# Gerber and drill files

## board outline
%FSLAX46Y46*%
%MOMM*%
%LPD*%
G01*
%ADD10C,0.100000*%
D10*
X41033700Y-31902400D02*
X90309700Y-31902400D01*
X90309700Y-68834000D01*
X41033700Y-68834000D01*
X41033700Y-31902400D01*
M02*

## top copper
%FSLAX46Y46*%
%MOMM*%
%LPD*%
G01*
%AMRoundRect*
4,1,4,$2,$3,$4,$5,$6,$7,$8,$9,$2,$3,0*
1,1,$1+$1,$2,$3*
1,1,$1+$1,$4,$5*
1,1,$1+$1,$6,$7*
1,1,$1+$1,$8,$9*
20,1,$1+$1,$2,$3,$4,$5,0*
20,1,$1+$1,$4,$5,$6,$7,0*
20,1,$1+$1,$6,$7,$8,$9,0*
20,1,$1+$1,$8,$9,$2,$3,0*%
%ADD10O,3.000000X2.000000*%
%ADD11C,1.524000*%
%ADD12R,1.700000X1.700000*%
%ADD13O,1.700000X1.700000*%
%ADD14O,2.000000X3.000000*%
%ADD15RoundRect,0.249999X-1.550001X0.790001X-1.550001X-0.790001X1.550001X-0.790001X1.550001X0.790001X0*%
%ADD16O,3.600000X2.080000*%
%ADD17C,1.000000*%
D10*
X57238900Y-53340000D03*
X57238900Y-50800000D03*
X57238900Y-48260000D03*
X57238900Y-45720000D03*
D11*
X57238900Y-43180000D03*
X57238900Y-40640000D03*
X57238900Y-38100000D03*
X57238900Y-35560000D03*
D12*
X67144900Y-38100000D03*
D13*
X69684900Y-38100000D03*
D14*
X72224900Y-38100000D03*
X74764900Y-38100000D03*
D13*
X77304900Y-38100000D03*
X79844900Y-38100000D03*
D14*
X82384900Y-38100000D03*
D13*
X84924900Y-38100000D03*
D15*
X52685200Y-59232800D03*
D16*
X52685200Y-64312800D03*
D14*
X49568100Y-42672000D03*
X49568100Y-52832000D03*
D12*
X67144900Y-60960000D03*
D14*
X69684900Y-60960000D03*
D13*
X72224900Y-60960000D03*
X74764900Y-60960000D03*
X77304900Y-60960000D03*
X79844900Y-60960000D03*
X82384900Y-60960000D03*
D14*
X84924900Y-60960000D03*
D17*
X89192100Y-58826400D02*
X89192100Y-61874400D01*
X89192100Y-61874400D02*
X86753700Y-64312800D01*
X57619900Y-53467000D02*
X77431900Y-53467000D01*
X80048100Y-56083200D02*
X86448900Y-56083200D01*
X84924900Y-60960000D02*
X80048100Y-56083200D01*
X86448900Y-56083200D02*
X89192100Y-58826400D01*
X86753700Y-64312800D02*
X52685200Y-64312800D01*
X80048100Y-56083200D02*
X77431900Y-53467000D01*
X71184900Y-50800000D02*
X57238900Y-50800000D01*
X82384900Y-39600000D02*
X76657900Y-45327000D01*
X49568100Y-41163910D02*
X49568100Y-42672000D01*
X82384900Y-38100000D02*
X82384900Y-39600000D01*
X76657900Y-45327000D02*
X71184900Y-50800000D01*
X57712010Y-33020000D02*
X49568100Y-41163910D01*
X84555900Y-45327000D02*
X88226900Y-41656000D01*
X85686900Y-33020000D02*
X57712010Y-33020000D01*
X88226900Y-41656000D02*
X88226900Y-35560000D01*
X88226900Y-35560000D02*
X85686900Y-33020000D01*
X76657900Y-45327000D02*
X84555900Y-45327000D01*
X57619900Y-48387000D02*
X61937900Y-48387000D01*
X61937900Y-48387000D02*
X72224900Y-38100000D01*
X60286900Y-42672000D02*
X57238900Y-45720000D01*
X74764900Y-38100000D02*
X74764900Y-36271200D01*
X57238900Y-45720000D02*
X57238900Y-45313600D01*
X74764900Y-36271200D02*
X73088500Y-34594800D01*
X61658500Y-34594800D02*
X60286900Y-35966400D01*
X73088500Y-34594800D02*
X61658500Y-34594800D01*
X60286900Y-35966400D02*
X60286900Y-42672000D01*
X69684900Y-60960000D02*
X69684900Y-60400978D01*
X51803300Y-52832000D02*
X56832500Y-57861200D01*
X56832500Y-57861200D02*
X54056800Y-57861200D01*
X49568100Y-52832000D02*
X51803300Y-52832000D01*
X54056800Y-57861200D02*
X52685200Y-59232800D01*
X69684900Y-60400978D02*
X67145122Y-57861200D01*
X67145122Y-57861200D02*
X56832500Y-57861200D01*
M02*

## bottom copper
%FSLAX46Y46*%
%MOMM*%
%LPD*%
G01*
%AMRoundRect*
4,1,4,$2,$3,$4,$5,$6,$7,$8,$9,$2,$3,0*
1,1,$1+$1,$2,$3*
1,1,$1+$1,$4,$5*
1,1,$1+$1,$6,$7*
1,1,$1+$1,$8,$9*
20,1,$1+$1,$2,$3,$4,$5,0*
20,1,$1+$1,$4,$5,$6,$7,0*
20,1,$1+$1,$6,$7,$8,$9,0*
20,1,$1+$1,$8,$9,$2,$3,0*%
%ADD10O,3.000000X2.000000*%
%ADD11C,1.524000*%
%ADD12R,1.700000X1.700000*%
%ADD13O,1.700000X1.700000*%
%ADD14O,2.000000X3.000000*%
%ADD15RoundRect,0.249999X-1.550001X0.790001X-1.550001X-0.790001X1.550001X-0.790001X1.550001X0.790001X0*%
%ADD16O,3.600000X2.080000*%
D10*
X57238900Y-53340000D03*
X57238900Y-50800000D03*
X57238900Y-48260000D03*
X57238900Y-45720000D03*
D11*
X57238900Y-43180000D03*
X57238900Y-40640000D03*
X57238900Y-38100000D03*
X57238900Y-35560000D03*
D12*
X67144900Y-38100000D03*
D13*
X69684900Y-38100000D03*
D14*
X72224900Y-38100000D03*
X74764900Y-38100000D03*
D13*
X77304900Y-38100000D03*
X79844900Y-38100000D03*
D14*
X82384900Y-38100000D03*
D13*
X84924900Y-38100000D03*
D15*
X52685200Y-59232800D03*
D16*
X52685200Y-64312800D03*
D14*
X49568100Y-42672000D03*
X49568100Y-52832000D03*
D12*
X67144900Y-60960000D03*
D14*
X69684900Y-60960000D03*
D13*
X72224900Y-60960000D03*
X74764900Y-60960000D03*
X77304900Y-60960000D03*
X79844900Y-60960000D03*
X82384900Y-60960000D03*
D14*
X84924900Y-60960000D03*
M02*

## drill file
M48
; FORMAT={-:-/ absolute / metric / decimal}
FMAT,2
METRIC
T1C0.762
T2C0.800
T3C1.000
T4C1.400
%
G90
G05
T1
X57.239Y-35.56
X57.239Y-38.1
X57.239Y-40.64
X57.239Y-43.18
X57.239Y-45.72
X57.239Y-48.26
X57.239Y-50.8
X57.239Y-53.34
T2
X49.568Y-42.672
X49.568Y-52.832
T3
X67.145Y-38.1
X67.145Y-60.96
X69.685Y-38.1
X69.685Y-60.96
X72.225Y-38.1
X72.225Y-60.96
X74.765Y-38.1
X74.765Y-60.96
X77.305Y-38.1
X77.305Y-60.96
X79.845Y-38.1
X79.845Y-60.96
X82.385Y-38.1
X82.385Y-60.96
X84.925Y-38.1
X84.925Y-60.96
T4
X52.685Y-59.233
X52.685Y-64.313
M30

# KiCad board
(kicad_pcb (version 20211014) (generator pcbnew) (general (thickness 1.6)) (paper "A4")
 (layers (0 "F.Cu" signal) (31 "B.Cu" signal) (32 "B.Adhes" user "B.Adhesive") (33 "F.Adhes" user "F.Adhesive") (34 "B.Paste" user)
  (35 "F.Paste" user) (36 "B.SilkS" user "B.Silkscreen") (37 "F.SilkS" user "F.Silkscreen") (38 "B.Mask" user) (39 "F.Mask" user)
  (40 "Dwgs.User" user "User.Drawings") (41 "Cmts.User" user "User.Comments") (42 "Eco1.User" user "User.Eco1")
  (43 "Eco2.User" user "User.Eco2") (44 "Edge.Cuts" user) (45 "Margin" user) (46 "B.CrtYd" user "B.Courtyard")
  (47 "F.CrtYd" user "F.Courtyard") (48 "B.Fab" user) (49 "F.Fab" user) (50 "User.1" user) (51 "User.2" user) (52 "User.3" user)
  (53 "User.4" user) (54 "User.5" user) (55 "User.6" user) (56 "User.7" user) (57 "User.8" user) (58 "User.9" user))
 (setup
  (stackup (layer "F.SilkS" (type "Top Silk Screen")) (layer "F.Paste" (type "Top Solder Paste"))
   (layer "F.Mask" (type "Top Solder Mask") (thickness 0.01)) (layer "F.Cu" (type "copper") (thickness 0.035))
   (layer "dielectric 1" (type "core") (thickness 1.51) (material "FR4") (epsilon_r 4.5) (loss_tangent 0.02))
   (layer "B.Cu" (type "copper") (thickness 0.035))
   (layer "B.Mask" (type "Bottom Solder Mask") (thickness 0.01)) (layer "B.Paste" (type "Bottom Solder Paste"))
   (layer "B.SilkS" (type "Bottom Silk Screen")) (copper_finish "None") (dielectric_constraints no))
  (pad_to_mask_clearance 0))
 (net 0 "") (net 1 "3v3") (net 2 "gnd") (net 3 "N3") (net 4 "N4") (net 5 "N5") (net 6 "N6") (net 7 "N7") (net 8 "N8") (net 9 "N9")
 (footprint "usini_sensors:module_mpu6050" (layer "F.Cu") (at 57.2389 35.56 180)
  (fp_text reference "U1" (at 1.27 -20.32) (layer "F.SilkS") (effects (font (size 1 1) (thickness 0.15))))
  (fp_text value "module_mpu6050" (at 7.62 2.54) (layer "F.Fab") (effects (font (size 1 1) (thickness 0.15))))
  (pad "1" thru_hole oval locked (at 0 -17.78 180) (size 3 2) (drill 0.762) (layers *.Cu *.Mask) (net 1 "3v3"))
  (pad "2" thru_hole oval locked (at 0 -15.24 180) (size 3 2) (drill 0.762) (layers *.Cu *.Mask) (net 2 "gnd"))
  (pad "3" thru_hole oval locked (at 0 -12.7 180) (size 3 2) (drill 0.762) (layers *.Cu *.Mask) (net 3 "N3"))
  (pad "4" thru_hole oval locked (at 0 -10.16 180) (size 3 2) (drill 0.762) (layers *.Cu *.Mask) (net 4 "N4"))
  (pad "5" thru_hole circle locked (at 0 -7.62 180) (size 1.524 1.524) (drill 0.762) (layers *.Cu *.Mask) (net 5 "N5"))
  (pad "6" thru_hole circle locked (at 0 -5.08 180) (size 1.524 1.524) (drill 0.762) (layers *.Cu *.Mask) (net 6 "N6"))
  (pad "7" thru_hole circle locked (at 0 -2.54 180) (size 1.524 1.524) (drill 0.762) (layers *.Cu *.Mask) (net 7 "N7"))
  (pad "8" thru_hole circle locked (at 0 0 180) (size 1.524 1.524) (drill 0.762) (layers *.Cu *.Mask) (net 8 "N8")))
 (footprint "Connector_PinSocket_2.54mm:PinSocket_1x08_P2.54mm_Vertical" (layer "F.Cu") (at 67.1449 38.1 90)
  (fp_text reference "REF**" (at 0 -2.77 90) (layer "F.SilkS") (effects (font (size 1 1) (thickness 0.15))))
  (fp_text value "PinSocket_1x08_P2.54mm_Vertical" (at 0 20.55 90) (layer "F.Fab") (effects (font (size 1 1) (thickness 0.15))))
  (pad "1" thru_hole rect (at 0 0 90) (size 1.7 1.7) (drill 1) (layers *.Cu *.Mask))
  (pad "2" thru_hole oval (at 0 2.54 90) (size 1.7 1.7) (drill 1) (layers *.Cu *.Mask))
  (pad "3" thru_hole oval (at 0 5.08 90) (size 3 2) (drill 1) (layers *.Cu *.Mask))
  (pad "4" thru_hole oval (at 0 7.62 90) (size 3 2) (drill 1) (layers *.Cu *.Mask) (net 4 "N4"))
  (pad "5" thru_hole oval (at 0 10.16 90) (size 1.7 1.7) (drill 1) (layers *.Cu *.Mask))
  (pad "6" thru_hole oval (at 0 12.7 90) (size 1.7 1.7) (drill 1) (layers *.Cu *.Mask))
  (pad "7" thru_hole oval (at 0 15.24 90) (size 3 2) (drill 1) (layers *.Cu *.Mask) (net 2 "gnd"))
  (pad "8" thru_hole oval (at 0 17.78 90) (size 1.7 1.7) (drill 1) (layers *.Cu *.Mask)))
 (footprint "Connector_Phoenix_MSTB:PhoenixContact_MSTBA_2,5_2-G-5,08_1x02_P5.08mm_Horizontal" (layer "F.Cu") (at 52.6852 59.2328 -90)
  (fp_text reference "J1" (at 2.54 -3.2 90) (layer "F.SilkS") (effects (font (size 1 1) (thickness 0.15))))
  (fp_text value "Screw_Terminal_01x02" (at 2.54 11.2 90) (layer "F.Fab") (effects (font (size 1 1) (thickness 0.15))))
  (pad "1" thru_hole roundrect (at 0 0 270) (size 2.08 3.6) (drill 1.4) (layers *.Cu *.Mask) (roundrect_rratio 0.120192) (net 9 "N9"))
  (pad "2" thru_hole oval (at 5.08 0 270) (size 2.08 3.6) (drill 1.4) (layers *.Cu *.Mask) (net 1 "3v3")))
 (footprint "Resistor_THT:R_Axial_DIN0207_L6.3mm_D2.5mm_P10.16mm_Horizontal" (layer "F.Cu") (at 49.5681 42.672 -90)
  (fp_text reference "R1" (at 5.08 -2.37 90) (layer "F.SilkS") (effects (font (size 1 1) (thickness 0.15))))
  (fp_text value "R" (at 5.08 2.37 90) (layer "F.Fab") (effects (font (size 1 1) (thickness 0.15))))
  (pad "1" thru_hole oval (at 0 0 270) (size 3 2) (drill 0.8) (layers *.Cu *.Mask) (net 2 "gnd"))
  (pad "2" thru_hole oval (at 10.16 0 270) (size 3 2) (drill 0.8) (layers *.Cu *.Mask) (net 9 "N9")))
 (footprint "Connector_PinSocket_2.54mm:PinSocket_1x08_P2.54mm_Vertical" (layer "F.Cu") (at 67.1449 60.96 90)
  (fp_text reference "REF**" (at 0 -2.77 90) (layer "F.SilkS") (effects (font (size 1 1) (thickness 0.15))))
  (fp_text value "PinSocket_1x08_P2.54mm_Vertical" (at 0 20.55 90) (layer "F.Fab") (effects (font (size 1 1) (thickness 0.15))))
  (pad "1" thru_hole rect (at 0 0 90) (size 1.7 1.7) (drill 1) (layers *.Cu *.Mask))
  (pad "2" thru_hole oval (at 0 2.54 90) (size 3 2) (drill 1) (layers *.Cu *.Mask) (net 9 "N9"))
  (pad "3" thru_hole oval (at 0 5.08 90) (size 1.7 1.7) (drill 1) (layers *.Cu *.Mask))
  (pad "4" thru_hole oval (at 0 7.62 90) (size 1.7 1.7) (drill 1) (layers *.Cu *.Mask))
  (pad "5" thru_hole oval (at 0 10.16 90) (size 1.7 1.7) (drill 1) (layers *.Cu *.Mask))
  (pad "6" thru_hole oval (at 0 12.7 90) (size 1.7 1.7) (drill 1) (layers *.Cu *.Mask))
  (pad "7" thru_hole oval (at 0 15.24 90) (size 1.7 1.7) (drill 1) (layers *.Cu *.Mask))
  (pad "8" thru_hole oval (at 0 17.78 90) (size 3 2) (drill 1) (layers *.Cu *.Mask) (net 1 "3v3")))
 (gr_rect (start 41.0337 68.834) (end 90.3097 31.9024) (layer "Edge.Cuts") (width 0.1) (fill none))
 (segment (start 89.1921 58.8264) (end 89.1921 61.8744) (width 1) (layer "F.Cu") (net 1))
 (segment (start 89.1921 61.8744) (end 86.7537 64.3128) (width 1) (layer "F.Cu") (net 1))
 (segment (start 57.6199 53.467) (end 77.4319 53.467) (width 1) (layer "F.Cu") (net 1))
 (segment (start 80.0481 56.0832) (end 86.4489 56.0832) (width 1) (layer "F.Cu") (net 1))
 (segment (start 84.9249 60.96) (end 80.0481 56.0832) (width 1) (layer "F.Cu") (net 1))
 (segment (start 86.4489 56.0832) (end 89.1921 58.8264) (width 1) (layer "F.Cu") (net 1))
 (segment (start 86.7537 64.3128) (end 52.6852 64.3128) (width 1) (layer "F.Cu") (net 1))
 (segment (start 80.0481 56.0832) (end 77.4319 53.467) (width 1) (layer "F.Cu") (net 1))
 (segment (start 71.1849 50.8) (end 57.2389 50.8) (width 1) (layer "F.Cu") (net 2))
 (segment (start 82.3849 39.6) (end 76.6579 45.327) (width 1) (layer "F.Cu") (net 2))
 (segment (start 49.5681 41.16391) (end 49.5681 42.672) (width 1) (layer "F.Cu") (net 2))
 (segment (start 82.3849 38.1) (end 82.3849 39.6) (width 1) (layer "F.Cu") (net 2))
 (segment (start 76.6579 45.327) (end 71.1849 50.8) (width 1) (layer "F.Cu") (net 2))
 (segment (start 57.71201 33.02) (end 49.5681 41.16391) (width 1) (layer "F.Cu") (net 2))
 (segment (start 84.5559 45.327) (end 88.2269 41.656) (width 1) (layer "F.Cu") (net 2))
 (segment (start 85.6869 33.02) (end 57.71201 33.02) (width 1) (layer "F.Cu") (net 2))
 (segment (start 88.2269 41.656) (end 88.2269 35.56) (width 1) (layer "F.Cu") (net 2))
 (segment (start 88.2269 35.56) (end 85.6869 33.02) (width 1) (layer "F.Cu") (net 2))
 (segment (start 76.6579 45.327) (end 84.5559 45.327) (width 1) (layer "F.Cu") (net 2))
 (segment (start 57.6199 48.387) (end 61.9379 48.387) (width 1) (layer "F.Cu") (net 3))
 (segment (start 61.9379 48.387) (end 72.2249 38.1) (width 1) (layer "F.Cu") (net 3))
 (segment (start 60.2869 42.672) (end 57.2389 45.72) (width 1) (layer "F.Cu") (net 4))
 (segment (start 74.7649 38.1) (end 74.7649 36.2712) (width 1) (layer "F.Cu") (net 4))
 (segment (start 57.2389 45.72) (end 57.2389 45.3136) (width 1) (layer "F.Cu") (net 4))
 (segment (start 74.7649 36.2712) (end 73.0885 34.5948) (width 1) (layer "F.Cu") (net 4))
 (segment (start 61.6585 34.5948) (end 60.2869 35.9664) (width 1) (layer "F.Cu") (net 4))
 (segment (start 73.0885 34.5948) (end 61.6585 34.5948) (width 1) (layer "F.Cu") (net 4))
 (segment (start 60.2869 35.9664) (end 60.2869 42.672) (width 1) (layer "F.Cu") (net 4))
 (segment (start 69.6849 60.96) (end 69.6849 60.400978) (width 1) (layer "F.Cu") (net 9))
 (segment (start 51.8033 52.832) (end 56.8325 57.8612) (width 1) (layer "F.Cu") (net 9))
 (segment (start 56.8325 57.8612) (end 54.0568 57.8612) (width 1) (layer "F.Cu") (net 9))
 (segment (start 49.5681 52.832) (end 51.8033 52.832) (width 1) (layer "F.Cu") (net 9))
 (segment (start 54.0568 57.8612) (end 52.6852 59.2328) (width 1) (layer "F.Cu") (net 9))
 (segment (start 69.6849 60.400978) (end 67.145122 57.8612) (width 1) (layer "F.Cu") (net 9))
 (segment (start 67.145122 57.8612) (end 56.8325 57.8612) (width 1) (layer "F.Cu") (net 9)))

